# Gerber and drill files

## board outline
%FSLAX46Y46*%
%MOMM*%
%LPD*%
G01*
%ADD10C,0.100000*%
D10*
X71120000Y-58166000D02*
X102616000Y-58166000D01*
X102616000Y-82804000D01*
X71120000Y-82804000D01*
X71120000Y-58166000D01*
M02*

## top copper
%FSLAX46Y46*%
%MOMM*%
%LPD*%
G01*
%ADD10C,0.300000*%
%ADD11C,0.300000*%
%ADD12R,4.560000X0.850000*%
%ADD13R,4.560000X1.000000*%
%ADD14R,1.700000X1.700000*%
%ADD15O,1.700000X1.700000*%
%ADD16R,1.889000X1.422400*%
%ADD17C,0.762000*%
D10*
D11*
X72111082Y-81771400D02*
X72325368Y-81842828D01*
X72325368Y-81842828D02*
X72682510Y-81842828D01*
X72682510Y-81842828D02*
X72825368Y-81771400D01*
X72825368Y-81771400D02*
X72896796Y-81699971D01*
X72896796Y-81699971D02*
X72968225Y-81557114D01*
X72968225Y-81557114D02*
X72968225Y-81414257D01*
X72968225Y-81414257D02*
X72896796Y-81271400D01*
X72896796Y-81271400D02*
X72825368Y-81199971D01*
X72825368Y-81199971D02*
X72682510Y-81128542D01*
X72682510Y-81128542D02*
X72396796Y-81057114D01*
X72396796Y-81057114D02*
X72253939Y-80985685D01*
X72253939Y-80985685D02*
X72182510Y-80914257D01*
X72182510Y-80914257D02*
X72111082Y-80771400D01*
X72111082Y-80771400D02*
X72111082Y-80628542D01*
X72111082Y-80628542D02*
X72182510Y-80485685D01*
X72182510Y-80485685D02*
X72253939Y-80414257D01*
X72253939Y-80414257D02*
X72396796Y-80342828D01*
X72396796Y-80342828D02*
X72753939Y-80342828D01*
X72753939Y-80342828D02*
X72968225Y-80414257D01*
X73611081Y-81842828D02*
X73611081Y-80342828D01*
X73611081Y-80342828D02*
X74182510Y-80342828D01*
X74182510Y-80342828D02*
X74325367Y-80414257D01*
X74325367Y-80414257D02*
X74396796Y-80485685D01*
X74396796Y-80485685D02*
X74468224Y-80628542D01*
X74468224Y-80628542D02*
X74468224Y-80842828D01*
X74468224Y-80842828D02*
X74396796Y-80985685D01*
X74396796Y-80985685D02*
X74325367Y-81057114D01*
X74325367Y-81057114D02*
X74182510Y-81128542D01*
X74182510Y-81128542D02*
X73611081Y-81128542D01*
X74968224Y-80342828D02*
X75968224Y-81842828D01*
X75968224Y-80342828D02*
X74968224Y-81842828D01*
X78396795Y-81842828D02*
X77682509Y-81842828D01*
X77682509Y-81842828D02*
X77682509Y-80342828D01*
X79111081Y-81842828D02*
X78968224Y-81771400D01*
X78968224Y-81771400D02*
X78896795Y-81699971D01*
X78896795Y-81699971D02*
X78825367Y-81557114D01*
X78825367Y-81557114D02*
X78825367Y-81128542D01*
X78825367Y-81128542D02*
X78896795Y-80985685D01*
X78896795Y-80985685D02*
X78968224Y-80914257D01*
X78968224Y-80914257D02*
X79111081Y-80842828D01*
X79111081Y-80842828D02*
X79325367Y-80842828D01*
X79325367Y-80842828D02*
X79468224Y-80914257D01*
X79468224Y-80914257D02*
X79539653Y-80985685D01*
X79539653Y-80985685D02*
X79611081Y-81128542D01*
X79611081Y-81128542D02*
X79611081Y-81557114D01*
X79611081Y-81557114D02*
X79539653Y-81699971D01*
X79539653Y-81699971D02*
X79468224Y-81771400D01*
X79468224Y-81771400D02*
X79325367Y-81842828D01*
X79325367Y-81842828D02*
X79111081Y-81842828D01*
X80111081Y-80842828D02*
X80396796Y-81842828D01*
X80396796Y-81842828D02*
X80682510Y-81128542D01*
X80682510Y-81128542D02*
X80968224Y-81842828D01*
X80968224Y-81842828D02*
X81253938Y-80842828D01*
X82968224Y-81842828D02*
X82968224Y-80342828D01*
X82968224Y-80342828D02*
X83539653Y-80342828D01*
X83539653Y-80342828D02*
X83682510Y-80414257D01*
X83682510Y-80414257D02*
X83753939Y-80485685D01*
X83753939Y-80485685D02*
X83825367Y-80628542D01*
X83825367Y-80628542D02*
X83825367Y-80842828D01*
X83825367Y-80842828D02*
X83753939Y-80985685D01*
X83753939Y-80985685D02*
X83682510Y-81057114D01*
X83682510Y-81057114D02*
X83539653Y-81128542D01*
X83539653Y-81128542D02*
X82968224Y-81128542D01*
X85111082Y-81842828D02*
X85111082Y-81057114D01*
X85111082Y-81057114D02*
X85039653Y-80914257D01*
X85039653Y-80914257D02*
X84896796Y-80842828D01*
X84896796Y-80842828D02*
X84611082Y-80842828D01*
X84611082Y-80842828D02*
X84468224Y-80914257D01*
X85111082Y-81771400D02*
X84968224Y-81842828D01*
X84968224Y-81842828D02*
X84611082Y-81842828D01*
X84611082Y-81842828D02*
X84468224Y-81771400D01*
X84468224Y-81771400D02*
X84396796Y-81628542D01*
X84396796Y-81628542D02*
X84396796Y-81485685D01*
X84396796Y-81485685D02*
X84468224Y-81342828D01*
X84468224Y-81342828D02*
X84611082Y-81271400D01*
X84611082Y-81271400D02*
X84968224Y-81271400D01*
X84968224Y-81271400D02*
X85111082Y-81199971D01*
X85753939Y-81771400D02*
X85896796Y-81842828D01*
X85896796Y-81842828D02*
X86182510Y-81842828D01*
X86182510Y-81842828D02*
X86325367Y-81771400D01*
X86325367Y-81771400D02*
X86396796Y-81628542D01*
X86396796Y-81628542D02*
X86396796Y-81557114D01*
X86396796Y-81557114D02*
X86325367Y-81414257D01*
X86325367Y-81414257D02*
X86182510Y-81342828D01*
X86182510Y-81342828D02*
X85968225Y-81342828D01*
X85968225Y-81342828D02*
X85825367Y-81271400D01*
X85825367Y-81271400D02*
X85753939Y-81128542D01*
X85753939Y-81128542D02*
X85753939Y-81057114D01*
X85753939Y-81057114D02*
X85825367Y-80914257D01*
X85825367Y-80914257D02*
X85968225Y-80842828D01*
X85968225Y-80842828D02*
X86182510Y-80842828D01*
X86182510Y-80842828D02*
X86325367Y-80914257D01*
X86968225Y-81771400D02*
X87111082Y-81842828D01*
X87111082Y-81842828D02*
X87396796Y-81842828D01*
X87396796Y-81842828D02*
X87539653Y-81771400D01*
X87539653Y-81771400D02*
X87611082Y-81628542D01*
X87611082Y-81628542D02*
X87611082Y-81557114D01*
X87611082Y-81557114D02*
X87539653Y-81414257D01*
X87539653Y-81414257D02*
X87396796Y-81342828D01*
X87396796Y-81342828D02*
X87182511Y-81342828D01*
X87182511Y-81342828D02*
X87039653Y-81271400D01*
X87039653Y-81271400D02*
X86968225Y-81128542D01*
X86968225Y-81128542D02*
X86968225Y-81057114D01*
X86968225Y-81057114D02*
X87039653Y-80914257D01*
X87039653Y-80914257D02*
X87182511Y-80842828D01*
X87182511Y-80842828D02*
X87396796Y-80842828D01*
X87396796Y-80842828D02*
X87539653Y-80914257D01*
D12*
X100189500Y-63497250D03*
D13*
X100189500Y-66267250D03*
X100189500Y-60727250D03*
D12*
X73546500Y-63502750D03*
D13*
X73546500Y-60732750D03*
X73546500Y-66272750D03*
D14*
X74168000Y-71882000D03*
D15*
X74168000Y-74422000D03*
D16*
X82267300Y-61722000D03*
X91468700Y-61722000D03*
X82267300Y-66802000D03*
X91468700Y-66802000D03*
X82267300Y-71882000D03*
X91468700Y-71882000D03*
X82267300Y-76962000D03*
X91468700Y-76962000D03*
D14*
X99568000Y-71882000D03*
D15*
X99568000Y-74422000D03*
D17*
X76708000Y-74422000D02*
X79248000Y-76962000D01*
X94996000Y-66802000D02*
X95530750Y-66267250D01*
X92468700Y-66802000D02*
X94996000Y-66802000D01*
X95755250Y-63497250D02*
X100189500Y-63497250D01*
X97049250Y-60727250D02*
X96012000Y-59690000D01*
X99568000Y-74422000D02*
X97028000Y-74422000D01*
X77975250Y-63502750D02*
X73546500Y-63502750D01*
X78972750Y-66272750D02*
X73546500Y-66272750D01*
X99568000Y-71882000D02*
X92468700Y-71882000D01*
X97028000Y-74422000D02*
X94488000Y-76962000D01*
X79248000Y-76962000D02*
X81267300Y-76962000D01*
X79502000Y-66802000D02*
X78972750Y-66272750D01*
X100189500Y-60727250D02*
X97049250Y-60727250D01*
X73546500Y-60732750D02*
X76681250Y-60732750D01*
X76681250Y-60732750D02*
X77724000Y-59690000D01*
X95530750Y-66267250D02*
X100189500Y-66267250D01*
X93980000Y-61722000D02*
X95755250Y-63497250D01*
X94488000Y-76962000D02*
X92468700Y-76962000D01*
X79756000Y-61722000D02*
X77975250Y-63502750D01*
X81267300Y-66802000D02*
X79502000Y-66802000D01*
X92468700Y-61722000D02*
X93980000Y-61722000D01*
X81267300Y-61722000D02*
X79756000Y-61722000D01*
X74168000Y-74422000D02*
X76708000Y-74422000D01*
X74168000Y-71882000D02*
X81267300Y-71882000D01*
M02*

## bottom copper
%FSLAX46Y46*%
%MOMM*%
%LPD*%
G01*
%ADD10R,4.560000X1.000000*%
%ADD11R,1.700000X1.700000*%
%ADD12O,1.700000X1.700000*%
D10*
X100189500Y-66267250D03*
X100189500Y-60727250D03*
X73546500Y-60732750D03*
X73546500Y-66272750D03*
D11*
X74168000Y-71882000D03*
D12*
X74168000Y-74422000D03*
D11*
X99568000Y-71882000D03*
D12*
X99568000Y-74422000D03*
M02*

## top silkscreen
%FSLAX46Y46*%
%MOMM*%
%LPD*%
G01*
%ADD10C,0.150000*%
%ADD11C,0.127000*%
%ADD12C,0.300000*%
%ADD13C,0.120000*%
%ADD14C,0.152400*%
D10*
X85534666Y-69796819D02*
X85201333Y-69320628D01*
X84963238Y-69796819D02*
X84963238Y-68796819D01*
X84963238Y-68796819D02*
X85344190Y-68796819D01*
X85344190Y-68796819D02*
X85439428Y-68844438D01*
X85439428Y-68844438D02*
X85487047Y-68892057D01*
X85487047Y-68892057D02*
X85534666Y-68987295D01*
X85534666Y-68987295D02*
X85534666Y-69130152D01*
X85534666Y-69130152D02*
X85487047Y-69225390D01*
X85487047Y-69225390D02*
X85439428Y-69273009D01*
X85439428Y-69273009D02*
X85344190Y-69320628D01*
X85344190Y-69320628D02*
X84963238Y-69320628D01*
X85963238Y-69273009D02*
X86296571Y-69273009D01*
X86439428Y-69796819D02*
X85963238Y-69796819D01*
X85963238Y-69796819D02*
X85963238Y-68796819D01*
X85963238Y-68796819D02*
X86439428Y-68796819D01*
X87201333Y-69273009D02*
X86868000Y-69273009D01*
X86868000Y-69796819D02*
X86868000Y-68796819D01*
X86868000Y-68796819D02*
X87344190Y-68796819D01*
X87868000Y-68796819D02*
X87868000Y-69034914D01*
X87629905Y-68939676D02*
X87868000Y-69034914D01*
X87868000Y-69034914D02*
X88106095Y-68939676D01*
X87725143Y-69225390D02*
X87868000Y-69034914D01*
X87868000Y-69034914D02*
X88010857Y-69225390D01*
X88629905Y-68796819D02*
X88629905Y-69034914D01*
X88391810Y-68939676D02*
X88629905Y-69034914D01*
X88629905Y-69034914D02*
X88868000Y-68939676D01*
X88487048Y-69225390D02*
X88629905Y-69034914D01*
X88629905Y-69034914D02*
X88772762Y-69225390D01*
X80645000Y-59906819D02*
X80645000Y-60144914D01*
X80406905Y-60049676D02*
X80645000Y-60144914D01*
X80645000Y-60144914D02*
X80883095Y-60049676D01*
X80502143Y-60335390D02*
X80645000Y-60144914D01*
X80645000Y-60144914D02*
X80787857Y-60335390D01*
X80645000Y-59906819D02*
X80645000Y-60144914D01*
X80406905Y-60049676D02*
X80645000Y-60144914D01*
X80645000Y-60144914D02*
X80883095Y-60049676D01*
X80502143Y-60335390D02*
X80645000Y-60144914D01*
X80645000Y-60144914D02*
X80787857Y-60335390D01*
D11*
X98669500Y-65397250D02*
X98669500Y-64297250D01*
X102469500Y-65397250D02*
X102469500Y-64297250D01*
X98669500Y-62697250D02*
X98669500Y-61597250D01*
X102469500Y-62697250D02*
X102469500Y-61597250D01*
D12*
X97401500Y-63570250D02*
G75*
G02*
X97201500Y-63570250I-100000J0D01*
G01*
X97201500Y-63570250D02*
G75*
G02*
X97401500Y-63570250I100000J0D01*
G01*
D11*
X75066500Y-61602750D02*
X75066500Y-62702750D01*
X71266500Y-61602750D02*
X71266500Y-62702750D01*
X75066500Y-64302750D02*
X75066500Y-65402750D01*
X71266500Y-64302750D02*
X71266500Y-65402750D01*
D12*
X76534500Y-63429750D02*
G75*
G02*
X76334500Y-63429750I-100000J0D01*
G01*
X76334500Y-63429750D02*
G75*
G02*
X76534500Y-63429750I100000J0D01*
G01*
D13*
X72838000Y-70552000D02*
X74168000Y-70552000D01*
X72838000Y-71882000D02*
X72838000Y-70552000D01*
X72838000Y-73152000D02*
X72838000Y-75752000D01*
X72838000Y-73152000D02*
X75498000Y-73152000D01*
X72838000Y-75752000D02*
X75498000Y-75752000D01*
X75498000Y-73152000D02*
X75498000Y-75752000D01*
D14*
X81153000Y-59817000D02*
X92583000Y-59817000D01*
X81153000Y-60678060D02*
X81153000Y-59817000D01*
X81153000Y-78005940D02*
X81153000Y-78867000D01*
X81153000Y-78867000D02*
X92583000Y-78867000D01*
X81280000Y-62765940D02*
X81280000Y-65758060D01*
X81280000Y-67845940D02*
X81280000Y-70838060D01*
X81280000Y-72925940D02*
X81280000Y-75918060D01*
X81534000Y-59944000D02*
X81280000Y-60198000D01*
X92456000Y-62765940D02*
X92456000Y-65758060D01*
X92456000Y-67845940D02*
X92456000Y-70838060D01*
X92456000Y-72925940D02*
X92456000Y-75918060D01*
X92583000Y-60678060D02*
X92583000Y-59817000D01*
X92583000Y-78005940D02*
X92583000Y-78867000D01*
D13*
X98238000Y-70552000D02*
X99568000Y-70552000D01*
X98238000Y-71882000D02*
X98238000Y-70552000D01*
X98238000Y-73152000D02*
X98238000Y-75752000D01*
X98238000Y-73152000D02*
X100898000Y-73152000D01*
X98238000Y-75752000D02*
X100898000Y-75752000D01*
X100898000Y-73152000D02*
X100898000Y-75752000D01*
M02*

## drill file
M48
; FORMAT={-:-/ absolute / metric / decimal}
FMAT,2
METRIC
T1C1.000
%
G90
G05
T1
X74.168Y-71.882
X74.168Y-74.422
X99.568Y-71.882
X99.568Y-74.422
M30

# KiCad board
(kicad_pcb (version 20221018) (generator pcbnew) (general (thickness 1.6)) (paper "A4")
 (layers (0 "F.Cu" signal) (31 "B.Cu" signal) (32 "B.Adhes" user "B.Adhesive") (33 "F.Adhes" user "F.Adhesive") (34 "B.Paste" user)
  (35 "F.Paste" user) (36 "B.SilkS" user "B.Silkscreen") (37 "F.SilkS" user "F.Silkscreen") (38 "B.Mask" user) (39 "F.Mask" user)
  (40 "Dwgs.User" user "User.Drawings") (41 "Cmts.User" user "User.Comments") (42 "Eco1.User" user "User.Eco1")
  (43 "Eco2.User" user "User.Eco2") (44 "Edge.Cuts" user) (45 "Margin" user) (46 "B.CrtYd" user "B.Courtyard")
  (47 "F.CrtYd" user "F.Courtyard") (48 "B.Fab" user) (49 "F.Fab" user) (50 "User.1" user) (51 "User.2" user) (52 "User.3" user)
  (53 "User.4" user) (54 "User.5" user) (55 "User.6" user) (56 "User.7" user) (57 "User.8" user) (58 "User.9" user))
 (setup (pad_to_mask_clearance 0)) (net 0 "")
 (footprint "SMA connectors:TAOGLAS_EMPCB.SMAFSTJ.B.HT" (layer "F.Cu") (at 100.1895 63.49725 90)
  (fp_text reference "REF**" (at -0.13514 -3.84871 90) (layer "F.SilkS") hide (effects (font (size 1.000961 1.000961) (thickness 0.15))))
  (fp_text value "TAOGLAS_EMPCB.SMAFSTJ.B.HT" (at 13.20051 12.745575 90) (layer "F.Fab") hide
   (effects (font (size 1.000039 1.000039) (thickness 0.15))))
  (fp_line (start -1.9 -1.52) (end -0.8 -1.52) (stroke (width 0.127) (type solid)) (layer "F.SilkS"))
  (fp_line (start -1.9 2.28) (end -0.8 2.28) (stroke (width 0.127) (type solid)) (layer "F.SilkS"))
  (fp_line (start 0.8 -1.52) (end 1.9 -1.52) (stroke (width 0.127) (type solid)) (layer "F.SilkS"))
  (fp_line (start 0.8 2.28) (end 1.9 2.28) (stroke (width 0.127) (type solid)) (layer "F.SilkS"))
  (fp_circle (center -0.073 -2.888) (end 0.027 -2.888) (stroke (width 0.3) (type solid)) (fill none) (layer "F.SilkS"))
  (pad "1" smd rect (at 0 0 90) (size 0.85 4.56) (layers "F.Cu" "F.Paste" "F.Mask") (solder_mask_margin 0.102))
  (pad "SH1" smd rect (at -2.77 0 90) (size 1 4.56) (layers "F.Cu" "F.Paste" "F.Mask") (solder_mask_margin 0.102))
  (pad "SH2" smd rect (at 2.77 0 90) (size 1 4.56) (layers "F.Cu" "F.Paste" "F.Mask") (solder_mask_margin 0.102))
  (pad "SH3" smd rect (at -2.77 0 90) (size 1 4.56) (layers "B.Cu" "B.Paste" "B.Mask") (solder_mask_margin 0.102))
  (pad "SH4" smd rect (at 2.77 0 90) (size 1 4.56) (layers "B.Cu" "B.Paste" "B.Mask") (solder_mask_margin 0.102)))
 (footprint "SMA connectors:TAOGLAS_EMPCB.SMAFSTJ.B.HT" (layer "F.Cu") (at 73.5465 63.50275 -90)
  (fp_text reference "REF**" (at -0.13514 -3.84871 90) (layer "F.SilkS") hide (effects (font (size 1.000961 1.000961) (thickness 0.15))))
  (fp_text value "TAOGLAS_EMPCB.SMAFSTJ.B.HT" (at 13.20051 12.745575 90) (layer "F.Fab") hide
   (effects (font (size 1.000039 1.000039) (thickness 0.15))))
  (fp_line (start -1.9 -1.52) (end -0.8 -1.52) (stroke (width 0.127) (type solid)) (layer "F.SilkS"))
  (fp_line (start -1.9 2.28) (end -0.8 2.28) (stroke (width 0.127) (type solid)) (layer "F.SilkS"))
  (fp_line (start 0.8 -1.52) (end 1.9 -1.52) (stroke (width 0.127) (type solid)) (layer "F.SilkS"))
  (fp_line (start 0.8 2.28) (end 1.9 2.28) (stroke (width 0.127) (type solid)) (layer "F.SilkS"))
  (fp_circle (center -0.073 -2.888) (end 0.027 -2.888) (stroke (width 0.3) (type solid)) (fill none) (layer "F.SilkS"))
  (pad "1" smd rect (at 0 0 270) (size 0.85 4.56) (layers "F.Cu" "F.Paste" "F.Mask") (solder_mask_margin 0.102))
  (pad "SH1" smd rect (at -2.77 0 270) (size 1 4.56) (layers "F.Cu" "F.Paste" "F.Mask") (solder_mask_margin 0.102))
  (pad "SH2" smd rect (at 2.77 0 270) (size 1 4.56) (layers "F.Cu" "F.Paste" "F.Mask") (solder_mask_margin 0.102))
  (pad "SH3" smd rect (at -2.77 0 270) (size 1 4.56) (layers "B.Cu" "B.Paste" "B.Mask") (solder_mask_margin 0.102))
  (pad "SH4" smd rect (at 2.77 0 270) (size 1 4.56) (layers "B.Cu" "B.Paste" "B.Mask") (solder_mask_margin 0.102)))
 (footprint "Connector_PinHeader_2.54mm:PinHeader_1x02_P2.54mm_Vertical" (layer "F.Cu") (at 74.168 71.882)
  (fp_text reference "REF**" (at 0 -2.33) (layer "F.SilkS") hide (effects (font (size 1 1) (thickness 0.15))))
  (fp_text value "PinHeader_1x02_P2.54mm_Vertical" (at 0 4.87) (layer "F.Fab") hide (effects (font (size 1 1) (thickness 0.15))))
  (fp_line (start -1.33 -1.33) (end 0 -1.33) (stroke (width 0.12) (type solid)) (layer "F.SilkS"))
  (fp_line (start -1.33 0) (end -1.33 -1.33) (stroke (width 0.12) (type solid)) (layer "F.SilkS"))
  (fp_line (start -1.33 1.27) (end -1.33 3.87) (stroke (width 0.12) (type solid)) (layer "F.SilkS"))
  (fp_line (start -1.33 1.27) (end 1.33 1.27) (stroke (width 0.12) (type solid)) (layer "F.SilkS"))
  (fp_line (start -1.33 3.87) (end 1.33 3.87) (stroke (width 0.12) (type solid)) (layer "F.SilkS"))
  (fp_line (start 1.33 1.27) (end 1.33 3.87) (stroke (width 0.12) (type solid)) (layer "F.SilkS"))
  (pad "1" thru_hole rect (at 0 0) (size 1.7 1.7) (drill 1) (layers "*.Cu" "*.Mask"))
  (pad "2" thru_hole oval (at 0 2.54) (size 1.7 1.7) (drill 1) (layers "*.Cu" "*.Mask")))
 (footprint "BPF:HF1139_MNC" (layer "F.Cu") (at 86.868 69.342)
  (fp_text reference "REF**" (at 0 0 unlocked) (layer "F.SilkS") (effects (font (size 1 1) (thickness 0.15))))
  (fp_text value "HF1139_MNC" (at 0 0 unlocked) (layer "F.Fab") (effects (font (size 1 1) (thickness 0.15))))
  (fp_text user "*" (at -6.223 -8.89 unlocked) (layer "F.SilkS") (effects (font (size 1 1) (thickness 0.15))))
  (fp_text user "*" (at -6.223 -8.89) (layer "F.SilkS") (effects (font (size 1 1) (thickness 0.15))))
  (fp_line (start -5.715 -9.525) (end 5.715 -9.525) (stroke (width 0.1524) (type solid)) (layer "F.SilkS"))
  (fp_line (start -5.715 -8.66394) (end -5.715 -9.525) (stroke (width 0.1524) (type solid)) (layer "F.SilkS"))
  (fp_line (start -5.715 8.66394) (end -5.715 9.525) (stroke (width 0.1524) (type solid)) (layer "F.SilkS"))
  (fp_line (start -5.715 9.525) (end 5.715 9.525) (stroke (width 0.1524) (type solid)) (layer "F.SilkS"))
  (fp_line (start -5.588 -6.57606) (end -5.588 -3.58394) (stroke (width 0.1524) (type solid)) (layer "F.SilkS"))
  (fp_line (start -5.588 -1.49606) (end -5.588 1.49606) (stroke (width 0.1524) (type solid)) (layer "F.SilkS"))
  (fp_line (start -5.588 3.58394) (end -5.588 6.57606) (stroke (width 0.1524) (type solid)) (layer "F.SilkS"))
  (fp_line (start -5.334 -9.398) (end -5.588 -9.144) (stroke (width 0.1524) (type solid)) (layer "F.SilkS"))
  (fp_line (start 5.588 -6.57606) (end 5.588 -3.58394) (stroke (width 0.1524) (type solid)) (layer "F.SilkS"))
  (fp_line (start 5.588 -1.49606) (end 5.588 1.49606) (stroke (width 0.1524) (type solid)) (layer "F.SilkS"))
  (fp_line (start 5.588 3.58394) (end 5.588 6.57606) (stroke (width 0.1524) (type solid)) (layer "F.SilkS"))
  (fp_line (start 5.715 -8.66394) (end 5.715 -9.525) (stroke (width 0.1524) (type solid)) (layer "F.SilkS"))
  (fp_line (start 5.715 8.66394) (end 5.715 9.525) (stroke (width 0.1524) (type solid)) (layer "F.SilkS"))
  (pad "1" smd rect (at -4.6007 -7.62) (size 1.889 1.4224) (layers "F.Cu" "F.Paste" "F.Mask"))
  (pad "2" smd rect (at 4.6007 -7.62) (size 1.889 1.4224) (layers "F.Cu" "F.Paste" "F.Mask"))
  (pad "3" smd rect (at -4.6007 -2.54) (size 1.889 1.4224) (layers "F.Cu" "F.Paste" "F.Mask"))
  (pad "4" smd rect (at 4.6007 -2.54) (size 1.889 1.4224) (layers "F.Cu" "F.Paste" "F.Mask"))
  (pad "5" smd rect (at -4.6007 2.54) (size 1.889 1.4224) (layers "F.Cu" "F.Paste" "F.Mask"))
  (pad "6" smd rect (at 4.6007 2.54) (size 1.889 1.4224) (layers "F.Cu" "F.Paste" "F.Mask"))
  (pad "7" smd rect (at -4.6007 7.62) (size 1.889 1.4224) (layers "F.Cu" "F.Paste" "F.Mask"))
  (pad "8" smd rect (at 4.6007 7.62) (size 1.889 1.4224) (layers "F.Cu" "F.Paste" "F.Mask")))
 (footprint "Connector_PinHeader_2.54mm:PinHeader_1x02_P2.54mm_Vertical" (layer "F.Cu") (at 99.568 71.882)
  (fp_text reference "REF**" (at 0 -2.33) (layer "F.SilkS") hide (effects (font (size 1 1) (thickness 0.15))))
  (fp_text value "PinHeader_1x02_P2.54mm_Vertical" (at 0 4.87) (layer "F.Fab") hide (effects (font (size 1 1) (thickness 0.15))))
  (fp_line (start -1.33 -1.33) (end 0 -1.33) (stroke (width 0.12) (type solid)) (layer "F.SilkS"))
  (fp_line (start -1.33 0) (end -1.33 -1.33) (stroke (width 0.12) (type solid)) (layer "F.SilkS"))
  (fp_line (start -1.33 1.27) (end -1.33 3.87) (stroke (width 0.12) (type solid)) (layer "F.SilkS"))
  (fp_line (start -1.33 1.27) (end 1.33 1.27) (stroke (width 0.12) (type solid)) (layer "F.SilkS"))
  (fp_line (start -1.33 3.87) (end 1.33 3.87) (stroke (width 0.12) (type solid)) (layer "F.SilkS"))
  (fp_line (start 1.33 1.27) (end 1.33 3.87) (stroke (width 0.12) (type solid)) (layer "F.SilkS"))
  (pad "1" thru_hole rect (at 0 0) (size 1.7 1.7) (drill 1) (layers "*.Cu" "*.Mask"))
  (pad "2" thru_hole oval (at 0 2.54) (size 1.7 1.7) (drill 1) (layers "*.Cu" "*.Mask")))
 (gr_rect (start 71.12 58.166) (end 102.616 82.804) (stroke (width 0.1) (type default)) (fill none) (layer "Edge.Cuts"))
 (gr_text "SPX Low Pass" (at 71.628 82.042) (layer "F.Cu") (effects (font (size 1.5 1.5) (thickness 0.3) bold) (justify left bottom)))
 (segment (start 76.708 74.422) (end 79.248 76.962) (width 0.762) (layer "F.Cu") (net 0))
 (segment (start 94.996 66.802) (end 95.53075 66.26725) (width 0.762) (layer "F.Cu") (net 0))
 (segment (start 92.4687 66.802) (end 94.996 66.802) (width 0.762) (layer "F.Cu") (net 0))
 (segment (start 95.75525 63.49725) (end 100.1895 63.49725) (width 0.762) (layer "F.Cu") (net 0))
 (segment (start 97.04925 60.72725) (end 96.012 59.69) (width 0.762) (layer "F.Cu") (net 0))
 (segment (start 99.568 74.422) (end 97.028 74.422) (width 0.762) (layer "F.Cu") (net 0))
 (segment (start 77.97525 63.50275) (end 73.5465 63.50275) (width 0.762) (layer "F.Cu") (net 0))
 (segment (start 78.97275 66.27275) (end 73.5465 66.27275) (width 0.762) (layer "F.Cu") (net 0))
 (segment (start 99.568 71.882) (end 92.4687 71.882) (width 0.762) (layer "F.Cu") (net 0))
 (segment (start 97.028 74.422) (end 94.488 76.962) (width 0.762) (layer "F.Cu") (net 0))
 (segment (start 79.248 76.962) (end 81.2673 76.962) (width 0.762) (layer "F.Cu") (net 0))
 (segment (start 79.502 66.802) (end 78.97275 66.27275) (width 0.762) (layer "F.Cu") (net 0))
 (segment (start 100.1895 60.72725) (end 97.04925 60.72725) (width 0.762) (layer "F.Cu") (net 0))
 (segment (start 73.5465 60.73275) (end 76.68125 60.73275) (width 0.762) (layer "F.Cu") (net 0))
 (segment (start 76.68125 60.73275) (end 77.724 59.69) (width 0.762) (layer "F.Cu") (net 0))
 (segment (start 95.53075 66.26725) (end 100.1895 66.26725) (width 0.762) (layer "F.Cu") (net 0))
 (segment (start 93.98 61.722) (end 95.75525 63.49725) (width 0.762) (layer "F.Cu") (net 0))
 (segment (start 94.488 76.962) (end 92.4687 76.962) (width 0.762) (layer "F.Cu") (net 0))
 (segment (start 79.756 61.722) (end 77.97525 63.50275) (width 0.762) (layer "F.Cu") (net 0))
 (segment (start 81.2673 66.802) (end 79.502 66.802) (width 0.762) (layer "F.Cu") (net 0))
 (segment (start 92.4687 61.722) (end 93.98 61.722) (width 0.762) (layer "F.Cu") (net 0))
 (segment (start 81.2673 61.722) (end 79.756 61.722) (width 0.762) (layer "F.Cu") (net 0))
 (segment (start 74.168 74.422) (end 76.708 74.422) (width 0.762) (layer "F.Cu") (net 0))
 (segment (start 74.168 71.882) (end 81.2673 71.882) (width 0.762) (layer "F.Cu") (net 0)))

